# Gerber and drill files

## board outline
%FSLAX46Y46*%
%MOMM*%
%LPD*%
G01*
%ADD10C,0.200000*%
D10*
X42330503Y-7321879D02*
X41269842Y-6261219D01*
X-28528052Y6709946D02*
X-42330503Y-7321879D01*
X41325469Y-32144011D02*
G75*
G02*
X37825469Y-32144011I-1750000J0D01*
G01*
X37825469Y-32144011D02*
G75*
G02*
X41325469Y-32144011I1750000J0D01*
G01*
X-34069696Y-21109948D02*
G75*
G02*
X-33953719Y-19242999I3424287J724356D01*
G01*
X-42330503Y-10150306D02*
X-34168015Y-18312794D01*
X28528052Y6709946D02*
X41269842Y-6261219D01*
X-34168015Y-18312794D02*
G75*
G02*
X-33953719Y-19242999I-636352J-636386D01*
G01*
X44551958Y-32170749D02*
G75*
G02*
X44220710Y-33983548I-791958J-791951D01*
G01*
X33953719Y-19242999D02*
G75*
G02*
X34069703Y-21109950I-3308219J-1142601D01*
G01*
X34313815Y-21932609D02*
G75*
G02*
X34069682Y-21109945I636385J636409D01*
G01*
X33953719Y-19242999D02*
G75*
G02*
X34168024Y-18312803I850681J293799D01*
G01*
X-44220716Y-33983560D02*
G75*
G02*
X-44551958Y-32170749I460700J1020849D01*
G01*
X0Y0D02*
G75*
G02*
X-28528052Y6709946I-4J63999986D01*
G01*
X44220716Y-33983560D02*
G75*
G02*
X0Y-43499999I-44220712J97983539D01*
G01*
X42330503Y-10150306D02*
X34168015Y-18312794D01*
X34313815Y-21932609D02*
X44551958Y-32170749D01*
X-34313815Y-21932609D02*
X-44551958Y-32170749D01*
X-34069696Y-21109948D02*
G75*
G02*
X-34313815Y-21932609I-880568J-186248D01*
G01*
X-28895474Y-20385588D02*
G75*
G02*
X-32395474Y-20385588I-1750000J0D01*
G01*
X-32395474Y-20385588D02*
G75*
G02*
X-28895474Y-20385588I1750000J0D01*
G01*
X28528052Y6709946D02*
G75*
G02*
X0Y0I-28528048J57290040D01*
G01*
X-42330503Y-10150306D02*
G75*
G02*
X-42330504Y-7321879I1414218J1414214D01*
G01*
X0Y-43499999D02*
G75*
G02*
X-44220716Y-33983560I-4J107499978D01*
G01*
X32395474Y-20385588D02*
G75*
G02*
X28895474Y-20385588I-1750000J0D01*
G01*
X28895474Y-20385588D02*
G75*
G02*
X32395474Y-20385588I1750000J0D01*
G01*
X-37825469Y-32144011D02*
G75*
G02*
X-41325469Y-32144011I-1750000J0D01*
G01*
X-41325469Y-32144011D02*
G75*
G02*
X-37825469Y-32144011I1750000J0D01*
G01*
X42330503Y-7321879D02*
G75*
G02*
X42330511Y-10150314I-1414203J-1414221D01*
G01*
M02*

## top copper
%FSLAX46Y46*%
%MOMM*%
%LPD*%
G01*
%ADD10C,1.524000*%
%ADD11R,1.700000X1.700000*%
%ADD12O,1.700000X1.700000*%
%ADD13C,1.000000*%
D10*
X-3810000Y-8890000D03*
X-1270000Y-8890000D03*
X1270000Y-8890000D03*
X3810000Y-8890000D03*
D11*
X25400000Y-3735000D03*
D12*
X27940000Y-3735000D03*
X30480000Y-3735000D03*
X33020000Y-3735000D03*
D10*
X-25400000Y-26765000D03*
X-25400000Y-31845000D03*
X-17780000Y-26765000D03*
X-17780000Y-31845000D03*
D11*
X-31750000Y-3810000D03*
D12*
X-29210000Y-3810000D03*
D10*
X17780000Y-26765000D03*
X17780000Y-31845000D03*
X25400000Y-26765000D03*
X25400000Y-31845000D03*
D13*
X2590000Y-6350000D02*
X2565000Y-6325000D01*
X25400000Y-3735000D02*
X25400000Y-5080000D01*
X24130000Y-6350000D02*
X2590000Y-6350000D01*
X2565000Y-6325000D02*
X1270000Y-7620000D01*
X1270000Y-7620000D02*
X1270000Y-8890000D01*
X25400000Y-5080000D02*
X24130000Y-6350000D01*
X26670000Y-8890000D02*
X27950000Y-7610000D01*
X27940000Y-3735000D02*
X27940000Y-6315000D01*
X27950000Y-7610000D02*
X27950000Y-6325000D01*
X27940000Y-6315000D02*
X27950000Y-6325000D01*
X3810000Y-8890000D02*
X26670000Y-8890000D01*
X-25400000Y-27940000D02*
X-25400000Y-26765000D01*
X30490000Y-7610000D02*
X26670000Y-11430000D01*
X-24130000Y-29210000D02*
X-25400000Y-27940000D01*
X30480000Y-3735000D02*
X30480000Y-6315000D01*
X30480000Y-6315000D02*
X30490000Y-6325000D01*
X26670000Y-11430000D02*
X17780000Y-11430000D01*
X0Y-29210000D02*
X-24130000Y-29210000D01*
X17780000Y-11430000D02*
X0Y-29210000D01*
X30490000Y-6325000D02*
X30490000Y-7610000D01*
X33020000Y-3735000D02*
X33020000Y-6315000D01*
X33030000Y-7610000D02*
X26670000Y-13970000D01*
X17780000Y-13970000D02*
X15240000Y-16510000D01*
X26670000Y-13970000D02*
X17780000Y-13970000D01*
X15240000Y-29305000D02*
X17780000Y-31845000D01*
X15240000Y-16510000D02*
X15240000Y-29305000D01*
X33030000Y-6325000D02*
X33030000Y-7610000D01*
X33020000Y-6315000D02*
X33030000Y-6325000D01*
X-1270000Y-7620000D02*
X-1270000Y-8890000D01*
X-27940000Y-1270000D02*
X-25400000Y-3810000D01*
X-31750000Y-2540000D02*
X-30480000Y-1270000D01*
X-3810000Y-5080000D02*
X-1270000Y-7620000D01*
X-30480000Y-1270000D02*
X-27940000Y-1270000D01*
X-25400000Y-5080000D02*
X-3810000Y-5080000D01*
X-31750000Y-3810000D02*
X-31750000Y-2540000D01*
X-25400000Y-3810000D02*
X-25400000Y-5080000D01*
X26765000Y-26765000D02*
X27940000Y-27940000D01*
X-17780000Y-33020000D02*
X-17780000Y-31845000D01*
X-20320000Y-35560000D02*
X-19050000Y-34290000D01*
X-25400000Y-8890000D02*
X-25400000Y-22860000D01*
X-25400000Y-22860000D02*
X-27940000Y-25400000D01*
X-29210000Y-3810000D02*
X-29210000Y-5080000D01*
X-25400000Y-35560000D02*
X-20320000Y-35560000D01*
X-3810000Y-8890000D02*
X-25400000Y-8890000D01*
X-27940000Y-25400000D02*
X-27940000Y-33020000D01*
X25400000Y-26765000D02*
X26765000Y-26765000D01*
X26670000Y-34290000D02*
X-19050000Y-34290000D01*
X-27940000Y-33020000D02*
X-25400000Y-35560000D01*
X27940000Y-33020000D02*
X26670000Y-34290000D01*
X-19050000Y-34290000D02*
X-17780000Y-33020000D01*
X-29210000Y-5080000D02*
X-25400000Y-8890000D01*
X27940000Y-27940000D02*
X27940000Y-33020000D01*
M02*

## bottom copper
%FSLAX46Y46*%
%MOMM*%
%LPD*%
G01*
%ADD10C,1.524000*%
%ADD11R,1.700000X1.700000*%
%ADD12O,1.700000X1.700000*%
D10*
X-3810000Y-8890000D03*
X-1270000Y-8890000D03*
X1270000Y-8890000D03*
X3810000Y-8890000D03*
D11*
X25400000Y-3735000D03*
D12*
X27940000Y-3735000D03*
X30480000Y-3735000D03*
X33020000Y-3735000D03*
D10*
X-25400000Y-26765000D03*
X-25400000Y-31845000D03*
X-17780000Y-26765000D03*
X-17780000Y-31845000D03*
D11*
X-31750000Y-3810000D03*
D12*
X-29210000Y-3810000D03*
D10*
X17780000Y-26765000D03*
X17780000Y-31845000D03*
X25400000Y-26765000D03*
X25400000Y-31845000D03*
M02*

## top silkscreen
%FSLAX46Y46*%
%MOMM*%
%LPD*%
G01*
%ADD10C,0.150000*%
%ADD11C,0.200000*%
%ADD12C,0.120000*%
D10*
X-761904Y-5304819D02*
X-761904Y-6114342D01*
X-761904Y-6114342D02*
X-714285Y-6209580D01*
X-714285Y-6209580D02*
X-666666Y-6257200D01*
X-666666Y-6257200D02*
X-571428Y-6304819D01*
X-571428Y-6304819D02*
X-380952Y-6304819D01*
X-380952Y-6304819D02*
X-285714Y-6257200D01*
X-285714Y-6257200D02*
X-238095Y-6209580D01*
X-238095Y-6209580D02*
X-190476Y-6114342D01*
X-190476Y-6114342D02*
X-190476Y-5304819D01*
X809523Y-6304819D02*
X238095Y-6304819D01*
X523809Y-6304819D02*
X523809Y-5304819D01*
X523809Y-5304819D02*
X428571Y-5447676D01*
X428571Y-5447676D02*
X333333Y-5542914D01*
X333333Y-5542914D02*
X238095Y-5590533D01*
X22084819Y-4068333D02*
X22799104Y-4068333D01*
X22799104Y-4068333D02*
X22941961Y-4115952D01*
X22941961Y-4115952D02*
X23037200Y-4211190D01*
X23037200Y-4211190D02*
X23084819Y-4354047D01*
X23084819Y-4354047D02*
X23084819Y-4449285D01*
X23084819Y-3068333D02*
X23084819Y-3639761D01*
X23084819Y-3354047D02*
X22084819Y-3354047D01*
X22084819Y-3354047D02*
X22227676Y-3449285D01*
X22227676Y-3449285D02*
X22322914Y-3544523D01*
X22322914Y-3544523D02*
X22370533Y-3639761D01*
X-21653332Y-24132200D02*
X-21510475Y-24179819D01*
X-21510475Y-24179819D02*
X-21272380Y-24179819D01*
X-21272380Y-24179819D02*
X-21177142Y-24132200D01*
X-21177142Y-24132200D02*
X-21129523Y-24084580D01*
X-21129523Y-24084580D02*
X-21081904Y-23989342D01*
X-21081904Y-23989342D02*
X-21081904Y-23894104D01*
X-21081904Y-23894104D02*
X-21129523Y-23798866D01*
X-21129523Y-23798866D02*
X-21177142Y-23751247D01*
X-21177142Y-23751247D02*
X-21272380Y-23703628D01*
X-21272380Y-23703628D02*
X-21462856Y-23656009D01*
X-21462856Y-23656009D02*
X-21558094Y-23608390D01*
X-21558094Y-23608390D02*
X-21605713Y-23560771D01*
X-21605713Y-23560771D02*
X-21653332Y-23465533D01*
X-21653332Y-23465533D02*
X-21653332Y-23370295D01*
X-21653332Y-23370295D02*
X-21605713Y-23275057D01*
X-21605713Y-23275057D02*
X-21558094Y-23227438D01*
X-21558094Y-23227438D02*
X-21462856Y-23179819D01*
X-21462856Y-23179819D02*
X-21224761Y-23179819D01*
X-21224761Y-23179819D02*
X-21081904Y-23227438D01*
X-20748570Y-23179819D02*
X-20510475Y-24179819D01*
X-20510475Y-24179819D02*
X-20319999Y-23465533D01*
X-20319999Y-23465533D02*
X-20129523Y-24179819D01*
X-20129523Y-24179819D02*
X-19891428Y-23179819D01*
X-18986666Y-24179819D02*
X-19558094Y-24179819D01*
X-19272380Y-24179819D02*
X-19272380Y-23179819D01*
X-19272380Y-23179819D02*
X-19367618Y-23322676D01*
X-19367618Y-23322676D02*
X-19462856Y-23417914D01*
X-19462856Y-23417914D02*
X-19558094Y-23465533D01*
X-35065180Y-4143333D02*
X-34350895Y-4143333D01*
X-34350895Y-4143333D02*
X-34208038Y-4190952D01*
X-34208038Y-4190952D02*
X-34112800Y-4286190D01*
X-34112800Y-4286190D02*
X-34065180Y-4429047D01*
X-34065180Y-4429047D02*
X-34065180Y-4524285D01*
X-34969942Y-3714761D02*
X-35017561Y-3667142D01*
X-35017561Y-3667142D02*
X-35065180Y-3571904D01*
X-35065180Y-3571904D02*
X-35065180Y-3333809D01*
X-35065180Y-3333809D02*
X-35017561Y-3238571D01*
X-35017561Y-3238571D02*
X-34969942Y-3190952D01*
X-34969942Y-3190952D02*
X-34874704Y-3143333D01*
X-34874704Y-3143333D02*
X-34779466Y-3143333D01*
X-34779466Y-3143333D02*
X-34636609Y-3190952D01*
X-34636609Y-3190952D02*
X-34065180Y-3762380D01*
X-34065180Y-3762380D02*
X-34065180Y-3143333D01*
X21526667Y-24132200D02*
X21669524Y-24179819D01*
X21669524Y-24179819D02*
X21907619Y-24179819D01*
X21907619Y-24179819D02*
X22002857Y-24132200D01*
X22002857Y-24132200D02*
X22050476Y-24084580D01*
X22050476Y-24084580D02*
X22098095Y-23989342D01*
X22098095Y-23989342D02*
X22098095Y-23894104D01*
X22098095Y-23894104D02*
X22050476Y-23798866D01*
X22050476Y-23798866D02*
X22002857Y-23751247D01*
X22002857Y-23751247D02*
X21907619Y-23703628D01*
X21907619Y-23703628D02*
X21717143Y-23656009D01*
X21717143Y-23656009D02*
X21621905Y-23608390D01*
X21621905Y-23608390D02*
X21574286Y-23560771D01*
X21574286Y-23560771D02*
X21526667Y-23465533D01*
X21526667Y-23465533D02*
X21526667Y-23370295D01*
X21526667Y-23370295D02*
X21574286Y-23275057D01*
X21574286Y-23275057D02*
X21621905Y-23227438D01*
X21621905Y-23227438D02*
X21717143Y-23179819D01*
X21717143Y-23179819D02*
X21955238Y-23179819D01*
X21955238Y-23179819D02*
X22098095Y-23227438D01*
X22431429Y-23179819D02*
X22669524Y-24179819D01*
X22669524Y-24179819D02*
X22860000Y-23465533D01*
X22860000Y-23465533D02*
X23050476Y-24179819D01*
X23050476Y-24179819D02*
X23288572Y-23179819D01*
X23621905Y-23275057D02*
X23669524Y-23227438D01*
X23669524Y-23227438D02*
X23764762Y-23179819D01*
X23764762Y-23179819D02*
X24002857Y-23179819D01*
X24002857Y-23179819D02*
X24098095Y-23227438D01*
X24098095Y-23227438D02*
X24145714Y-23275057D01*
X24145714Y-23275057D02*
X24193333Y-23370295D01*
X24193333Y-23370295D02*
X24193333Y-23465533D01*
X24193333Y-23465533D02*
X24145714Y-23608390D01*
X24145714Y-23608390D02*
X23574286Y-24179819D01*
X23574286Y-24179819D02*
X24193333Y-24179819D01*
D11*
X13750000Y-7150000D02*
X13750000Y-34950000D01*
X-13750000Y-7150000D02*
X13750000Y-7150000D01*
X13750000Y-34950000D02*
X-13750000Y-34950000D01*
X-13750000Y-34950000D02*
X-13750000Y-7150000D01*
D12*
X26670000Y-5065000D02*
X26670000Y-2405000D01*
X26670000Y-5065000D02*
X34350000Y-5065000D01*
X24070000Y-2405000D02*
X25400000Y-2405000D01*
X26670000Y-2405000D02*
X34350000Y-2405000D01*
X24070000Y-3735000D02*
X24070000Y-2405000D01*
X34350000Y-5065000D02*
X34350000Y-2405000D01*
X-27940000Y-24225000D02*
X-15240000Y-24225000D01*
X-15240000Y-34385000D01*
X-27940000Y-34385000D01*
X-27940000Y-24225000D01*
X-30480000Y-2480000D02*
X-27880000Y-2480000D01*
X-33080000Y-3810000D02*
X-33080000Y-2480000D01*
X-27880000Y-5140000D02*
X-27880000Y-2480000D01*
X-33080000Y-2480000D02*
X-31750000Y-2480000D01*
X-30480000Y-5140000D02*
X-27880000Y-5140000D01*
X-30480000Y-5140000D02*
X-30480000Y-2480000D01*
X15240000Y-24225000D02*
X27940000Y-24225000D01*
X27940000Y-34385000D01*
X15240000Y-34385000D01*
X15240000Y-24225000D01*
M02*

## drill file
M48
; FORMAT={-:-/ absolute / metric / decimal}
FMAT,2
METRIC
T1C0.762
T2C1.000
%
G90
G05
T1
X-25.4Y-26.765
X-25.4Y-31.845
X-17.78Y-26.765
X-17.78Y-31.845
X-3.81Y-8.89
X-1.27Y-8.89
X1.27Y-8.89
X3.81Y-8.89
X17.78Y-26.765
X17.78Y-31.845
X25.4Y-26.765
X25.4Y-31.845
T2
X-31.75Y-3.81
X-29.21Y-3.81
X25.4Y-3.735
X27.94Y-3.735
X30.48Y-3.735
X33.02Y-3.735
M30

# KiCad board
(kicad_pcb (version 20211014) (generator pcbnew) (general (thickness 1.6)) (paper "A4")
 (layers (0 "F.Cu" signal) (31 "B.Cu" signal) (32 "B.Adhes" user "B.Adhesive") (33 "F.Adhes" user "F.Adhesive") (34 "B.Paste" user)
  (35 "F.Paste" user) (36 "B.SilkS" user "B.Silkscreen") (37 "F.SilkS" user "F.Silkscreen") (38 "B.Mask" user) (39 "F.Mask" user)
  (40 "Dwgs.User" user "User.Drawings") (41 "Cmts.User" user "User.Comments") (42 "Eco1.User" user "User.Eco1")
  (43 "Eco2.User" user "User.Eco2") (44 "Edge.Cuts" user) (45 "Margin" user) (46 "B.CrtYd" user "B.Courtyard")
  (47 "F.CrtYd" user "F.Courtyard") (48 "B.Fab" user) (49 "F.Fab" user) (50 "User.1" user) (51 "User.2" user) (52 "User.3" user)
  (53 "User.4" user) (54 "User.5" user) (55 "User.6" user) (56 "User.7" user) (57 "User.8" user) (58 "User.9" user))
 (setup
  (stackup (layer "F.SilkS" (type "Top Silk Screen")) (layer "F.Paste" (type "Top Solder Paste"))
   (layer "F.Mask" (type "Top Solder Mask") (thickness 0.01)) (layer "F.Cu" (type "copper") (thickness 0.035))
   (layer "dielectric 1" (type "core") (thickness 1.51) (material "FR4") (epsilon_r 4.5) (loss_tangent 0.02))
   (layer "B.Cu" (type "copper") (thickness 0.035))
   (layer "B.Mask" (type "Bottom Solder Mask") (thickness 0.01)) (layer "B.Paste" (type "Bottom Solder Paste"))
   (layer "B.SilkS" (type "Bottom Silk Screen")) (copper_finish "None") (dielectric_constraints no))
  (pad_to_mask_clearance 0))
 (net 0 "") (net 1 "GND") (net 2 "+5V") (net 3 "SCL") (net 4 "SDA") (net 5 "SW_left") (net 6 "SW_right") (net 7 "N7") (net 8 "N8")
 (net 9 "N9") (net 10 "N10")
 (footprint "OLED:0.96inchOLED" (layer "F.Cu") (at 0 6.35)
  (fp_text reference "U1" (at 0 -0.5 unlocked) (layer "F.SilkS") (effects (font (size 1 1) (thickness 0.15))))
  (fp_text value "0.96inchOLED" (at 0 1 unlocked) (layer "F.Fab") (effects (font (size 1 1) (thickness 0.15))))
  (fp_line (start 13.75 0.8) (end 13.75 28.6) (layer "F.SilkS") (width 0.2))
  (fp_line (start -13.75 0.8) (end 13.75 0.8) (layer "F.SilkS") (width 0.2))
  (fp_line (start 13.75 28.6) (end -13.75 28.6) (layer "F.SilkS") (width 0.2))
  (fp_line (start -13.75 28.6) (end -13.75 0.8) (layer "F.SilkS") (width 0.2))
  (pad "1" thru_hole circle (at -3.81 2.54) (size 1.524 1.524) (drill 0.762) (layers *.Cu *.Mask) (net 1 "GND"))
  (pad "2" thru_hole circle (at -1.27 2.54) (size 1.524 1.524) (drill 0.762) (layers *.Cu *.Mask) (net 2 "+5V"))
  (pad "3" thru_hole circle (at 1.27 2.54) (size 1.524 1.524) (drill 0.762) (layers *.Cu *.Mask) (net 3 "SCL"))
  (pad "4" thru_hole circle (at 3.81 2.54) (size 1.524 1.524) (drill 0.762) (layers *.Cu *.Mask) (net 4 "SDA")))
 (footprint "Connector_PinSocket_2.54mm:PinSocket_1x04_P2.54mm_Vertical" (layer "F.Cu") (at 25.4 3.735 90)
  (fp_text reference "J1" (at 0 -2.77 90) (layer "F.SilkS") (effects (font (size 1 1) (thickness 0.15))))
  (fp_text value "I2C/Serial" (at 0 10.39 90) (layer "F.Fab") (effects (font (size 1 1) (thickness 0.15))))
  (fp_line (start -1.33 1.27) (end 1.33 1.27) (layer "F.SilkS") (width 0.12))
  (fp_line (start -1.33 1.27) (end -1.33 8.95) (layer "F.SilkS") (width 0.12))
  (fp_line (start 1.33 -1.33) (end 1.33 0) (layer "F.SilkS") (width 0.12))
  (fp_line (start 1.33 1.27) (end 1.33 8.95) (layer "F.SilkS") (width 0.12))
  (fp_line (start 0 -1.33) (end 1.33 -1.33) (layer "F.SilkS") (width 0.12))
  (fp_line (start -1.33 8.95) (end 1.33 8.95) (layer "F.SilkS") (width 0.12))
  (pad "1" thru_hole rect (at 0 0 90) (size 1.7 1.7) (drill 1) (layers *.Cu *.Mask) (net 3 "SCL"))
  (pad "2" thru_hole oval (at 0 2.54 90) (size 1.7 1.7) (drill 1) (layers *.Cu *.Mask) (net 4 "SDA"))
  (pad "3" thru_hole oval (at 0 5.08 90) (size 1.7 1.7) (drill 1) (layers *.Cu *.Mask) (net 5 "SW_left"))
  (pad "4" thru_hole oval (at 0 7.62 90) (size 1.7 1.7) (drill 1) (layers *.Cu *.Mask) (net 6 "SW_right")))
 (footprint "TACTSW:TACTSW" (layer "F.Cu") (at -20.32 24.225)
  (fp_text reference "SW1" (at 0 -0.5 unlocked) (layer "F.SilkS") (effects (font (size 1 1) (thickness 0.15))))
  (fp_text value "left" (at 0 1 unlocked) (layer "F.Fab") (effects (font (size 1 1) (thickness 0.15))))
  (fp_rect (start -7.62 0) (end 5.08 10.16) (layer "F.SilkS") (width 0.12) (fill none))
  (pad "1" thru_hole circle (at -5.08 2.54) (size 1.524 1.524) (drill 0.762) (layers *.Cu *.Mask) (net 5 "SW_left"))
  (pad "2" thru_hole circle (at -5.08 7.62) (size 1.524 1.524) (drill 0.762) (layers *.Cu *.Mask) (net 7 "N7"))
  (pad "3" thru_hole circle (at 2.54 2.54) (size 1.524 1.524) (drill 0.762) (layers *.Cu *.Mask) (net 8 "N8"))
  (pad "4" thru_hole circle (at 2.54 7.62) (size 1.524 1.524) (drill 0.762) (layers *.Cu *.Mask) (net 1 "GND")))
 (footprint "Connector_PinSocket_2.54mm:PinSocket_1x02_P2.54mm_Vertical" (layer "F.Cu") (at -31.75 3.81 90)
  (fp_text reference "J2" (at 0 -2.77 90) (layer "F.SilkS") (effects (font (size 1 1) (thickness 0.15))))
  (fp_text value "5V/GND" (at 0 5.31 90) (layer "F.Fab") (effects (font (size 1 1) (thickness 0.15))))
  (fp_line (start 1.33 1.27) (end 1.33 3.87) (layer "F.SilkS") (width 0.12))
  (fp_line (start 0 -1.33) (end 1.33 -1.33) (layer "F.SilkS") (width 0.12))
  (fp_line (start -1.33 3.87) (end 1.33 3.87) (layer "F.SilkS") (width 0.12))
  (fp_line (start 1.33 -1.33) (end 1.33 0) (layer "F.SilkS") (width 0.12))
  (fp_line (start -1.33 1.27) (end -1.33 3.87) (layer "F.SilkS") (width 0.12))
  (fp_line (start -1.33 1.27) (end 1.33 1.27) (layer "F.SilkS") (width 0.12))
  (pad "1" thru_hole rect (at 0 0 90) (size 1.7 1.7) (drill 1) (layers *.Cu *.Mask) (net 2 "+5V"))
  (pad "2" thru_hole oval (at 0 2.54 90) (size 1.7 1.7) (drill 1) (layers *.Cu *.Mask) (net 1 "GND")))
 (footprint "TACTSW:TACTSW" (layer "F.Cu") (at 22.86 24.225)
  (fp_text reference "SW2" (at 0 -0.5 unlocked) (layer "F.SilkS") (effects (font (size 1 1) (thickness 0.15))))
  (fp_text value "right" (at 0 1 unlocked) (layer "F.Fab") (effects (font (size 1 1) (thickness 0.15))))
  (fp_rect (start -7.62 0) (end 5.08 10.16) (layer "F.SilkS") (width 0.12) (fill none))
  (pad "1" thru_hole circle (at -5.08 2.54) (size 1.524 1.524) (drill 0.762) (layers *.Cu *.Mask) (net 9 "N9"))
  (pad "2" thru_hole circle (at -5.08 7.62) (size 1.524 1.524) (drill 0.762) (layers *.Cu *.Mask) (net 6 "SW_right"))
  (pad "3" thru_hole circle (at 2.54 2.54) (size 1.524 1.524) (drill 0.762) (layers *.Cu *.Mask) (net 1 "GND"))
  (pad "4" thru_hole circle (at 2.54 7.62) (size 1.524 1.524) (drill 0.762) (layers *.Cu *.Mask) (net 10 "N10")))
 (gr_line (start 42.330503 7.321879) (end 41.269842 6.261219) (layer "Edge.Cuts") (width 0.2))
 (gr_line (start -28.528052 -6.709946) (end -42.330503 7.321879) (layer "Edge.Cuts") (width 0.2))
 (gr_circle (center 39.575469 32.144011) (end 37.825469 32.144011) (layer "Edge.Cuts") (width 0.2) (fill none))
 (gr_arc (start -34.069696 21.109948) (mid -34.138737 20.168583) (end -33.953719 19.242999) (layer "Edge.Cuts") (width 0.2))
 (gr_line (start -42.330503 10.150306) (end -34.168015 18.312794) (layer "Edge.Cuts") (width 0.2))
 (gr_line (start 28.528052 -6.709946) (end 41.269842 6.261219) (layer "Edge.Cuts") (width 0.2))
 (gr_arc (start -34.168015 18.312794) (mid -33.927376 18.747145) (end -33.953719 19.242999) (layer "Edge.Cuts") (width 0.2))
 (gr_arc (start 44.551958 32.170749) (mid 44.861757 33.164024) (end 44.220716 33.98356) (layer "Edge.Cuts") (width 0.2))
 (gr_arc (start 33.953719 19.242999) (mid 34.13874 20.168582) (end 34.069696 21.109948) (layer "Edge.Cuts") (width 0.2))
 (gr_arc (start 34.313815 21.932609) (mid 34.087397 21.552246) (end 34.069696 21.109948) (layer "Edge.Cuts") (width 0.2))
 (gr_arc (start 33.953719 19.242999) (mid 33.927383 18.747145) (end 34.168015 18.312794) (layer "Edge.Cuts") (width 0.2))
 (gr_arc (start -44.220716 33.98356) (mid -44.861765 33.164022) (end -44.551958 32.170749) (layer "Edge.Cuts") (width 0.2))
 (gr_arc (start 0 0) (mid -14.653269 -1.700066) (end -28.528052 -6.709946) (layer "Edge.Cuts") (width 0.2))
 (gr_arc (start 44.220716 33.98356) (mid 22.616556 41.093964) (end 0 43.499999) (layer "Edge.Cuts") (width 0.2))
 (gr_line (start 42.330503 10.150306) (end 34.168015 18.312794) (layer "Edge.Cuts") (width 0.2))
 (gr_line (start 34.313815 21.932609) (end 44.551958 32.170749) (layer "Edge.Cuts") (width 0.2))
 (gr_line (start -34.313815 21.932609) (end -44.551958 32.170749) (layer "Edge.Cuts") (width 0.2))
 (gr_arc (start -34.069696 21.109948) (mid -34.087403 21.552242) (end -34.313815 21.932609) (layer "Edge.Cuts") (width 0.2))
 (gr_circle (center -30.645474 20.385588) (end -32.395474 20.385588) (layer "Edge.Cuts") (width 0.2) (fill none))
 (gr_arc (start 28.528052 -6.709946) (mid 14.653269 -1.700066) (end 0 0) (layer "Edge.Cuts") (width 0.2))
 (gr_arc (start -42.330503 10.150306) (mid -42.916288 8.736094) (end -42.330503 7.321879) (layer "Edge.Cuts") (width 0.2))
 (gr_arc (start 0 43.499999) (mid -22.616556 41.093964) (end -44.220716 33.98356) (layer "Edge.Cuts") (width 0.2))
 (gr_circle (center 30.645474 20.385588) (end 28.895474 20.385588) (layer "Edge.Cuts") (width 0.2) (fill none))
 (gr_circle (center -39.575469 32.144011) (end -41.325469 32.144011) (layer "Edge.Cuts") (width 0.2) (fill none))
 (gr_arc (start 42.330503 7.321879) (mid 42.916289 8.736093) (end 42.330503 10.150306) (layer "Edge.Cuts") (width 0.2))
 (segment (start 2.59 6.35) (end 2.565 6.325) (width 1) (layer "F.Cu") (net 3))
 (segment (start 25.4 3.735) (end 25.4 5.08) (width 1) (layer "F.Cu") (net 3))
 (segment (start 24.13 6.35) (end 2.59 6.35) (width 1) (layer "F.Cu") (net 3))
 (segment (start 2.565 6.325) (end 1.27 7.62) (width 1) (layer "F.Cu") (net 3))
 (segment (start 1.27 7.62) (end 1.27 8.89) (width 1) (layer "F.Cu") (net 3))
 (segment (start 25.4 5.08) (end 24.13 6.35) (width 1) (layer "F.Cu") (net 3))
 (segment (start 26.67 8.89) (end 27.95 7.61) (width 1) (layer "F.Cu") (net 4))
 (segment (start 27.94 3.735) (end 27.94 6.315) (width 1) (layer "F.Cu") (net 4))
 (segment (start 27.95 7.61) (end 27.95 6.325) (width 1) (layer "F.Cu") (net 4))
 (segment (start 27.94 6.315) (end 27.95 6.325) (width 1) (layer "F.Cu") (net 4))
 (segment (start 3.81 8.89) (end 26.67 8.89) (width 1) (layer "F.Cu") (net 4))
 (segment (start -25.4 27.94) (end -25.4 26.765) (width 1) (layer "F.Cu") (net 5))
 (segment (start 30.49 7.61) (end 26.67 11.43) (width 1) (layer "F.Cu") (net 5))
 (segment (start -24.13 29.21) (end -25.4 27.94) (width 1) (layer "F.Cu") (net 5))
 (segment (start 30.48 3.735) (end 30.48 6.315) (width 1) (layer "F.Cu") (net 5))
 (segment (start 30.48 6.315) (end 30.49 6.325) (width 1) (layer "F.Cu") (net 5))
 (segment (start 26.67 11.43) (end 17.78 11.43) (width 1) (layer "F.Cu") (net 5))
 (segment (start 0 29.21) (end -24.13 29.21) (width 1) (layer "F.Cu") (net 5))
 (segment (start 17.78 11.43) (end 0 29.21) (width 1) (layer "F.Cu") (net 5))
 (segment (start 30.49 6.325) (end 30.49 7.61) (width 1) (layer "F.Cu") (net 5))
 (segment (start 33.02 3.735) (end 33.02 6.315) (width 1) (layer "F.Cu") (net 6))
 (segment (start 33.03 7.61) (end 26.67 13.97) (width 1) (layer "F.Cu") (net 6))
 (segment (start 17.78 13.97) (end 15.24 16.51) (width 1) (layer "F.Cu") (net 6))
 (segment (start 26.67 13.97) (end 17.78 13.97) (width 1) (layer "F.Cu") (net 6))
 (segment (start 15.24 29.305) (end 17.78 31.845) (width 1) (layer "F.Cu") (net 6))
 (segment (start 15.24 16.51) (end 15.24 29.305) (width 1) (layer "F.Cu") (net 6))
 (segment (start 33.03 6.325) (end 33.03 7.61) (width 1) (layer "F.Cu") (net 6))
 (segment (start 33.02 6.315) (end 33.03 6.325) (width 1) (layer "F.Cu") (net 6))
 (segment (start -1.27 7.62) (end -1.27 8.89) (width 1) (layer "F.Cu") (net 2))
 (segment (start -27.94 1.27) (end -25.4 3.81) (width 1) (layer "F.Cu") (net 2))
 (segment (start -31.75 2.54) (end -30.48 1.27) (width 1) (layer "F.Cu") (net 2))
 (segment (start -3.81 5.08) (end -1.27 7.62) (width 1) (layer "F.Cu") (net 2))
 (segment (start -30.48 1.27) (end -27.94 1.27) (width 1) (layer "F.Cu") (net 2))
 (segment (start -25.4 5.08) (end -3.81 5.08) (width 1) (layer "F.Cu") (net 2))
 (segment (start -31.75 3.81) (end -31.75 2.54) (width 1) (layer "F.Cu") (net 2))
 (segment (start -25.4 3.81) (end -25.4 5.08) (width 1) (layer "F.Cu") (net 2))
 (segment (start 26.765 26.765) (end 27.94 27.94) (width 1) (layer "F.Cu") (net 1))
 (segment (start -17.78 33.02) (end -17.78 31.845) (width 1) (layer "F.Cu") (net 1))
 (segment (start -20.32 35.56) (end -19.05 34.29) (width 1) (layer "F.Cu") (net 1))
 (segment (start -25.4 8.89) (end -25.4 22.86) (width 1) (layer "F.Cu") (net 1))
 (segment (start -25.4 22.86) (end -27.94 25.4) (width 1) (layer "F.Cu") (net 1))
 (segment (start -29.21 3.81) (end -29.21 5.08) (width 1) (layer "F.Cu") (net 1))
 (segment (start -25.4 35.56) (end -20.32 35.56) (width 1) (layer "F.Cu") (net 1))
 (segment (start -3.81 8.89) (end -25.4 8.89) (width 1) (layer "F.Cu") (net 1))
 (segment (start -27.94 25.4) (end -27.94 33.02) (width 1) (layer "F.Cu") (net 1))
 (segment (start 25.4 26.765) (end 26.765 26.765) (width 1) (layer "F.Cu") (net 1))
 (segment (start 26.67 34.29) (end -19.05 34.29) (width 1) (layer "F.Cu") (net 1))
 (segment (start -27.94 33.02) (end -25.4 35.56) (width 1) (layer "F.Cu") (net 1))
 (segment (start 27.94 33.02) (end 26.67 34.29) (width 1) (layer "F.Cu") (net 1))
 (segment (start -19.05 34.29) (end -17.78 33.02) (width 1) (layer "F.Cu") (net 1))
 (segment (start -29.21 5.08) (end -25.4 8.89) (width 1) (layer "F.Cu") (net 1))
 (segment (start 27.94 27.94) (end 27.94 33.02) (width 1) (layer "F.Cu") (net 1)))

